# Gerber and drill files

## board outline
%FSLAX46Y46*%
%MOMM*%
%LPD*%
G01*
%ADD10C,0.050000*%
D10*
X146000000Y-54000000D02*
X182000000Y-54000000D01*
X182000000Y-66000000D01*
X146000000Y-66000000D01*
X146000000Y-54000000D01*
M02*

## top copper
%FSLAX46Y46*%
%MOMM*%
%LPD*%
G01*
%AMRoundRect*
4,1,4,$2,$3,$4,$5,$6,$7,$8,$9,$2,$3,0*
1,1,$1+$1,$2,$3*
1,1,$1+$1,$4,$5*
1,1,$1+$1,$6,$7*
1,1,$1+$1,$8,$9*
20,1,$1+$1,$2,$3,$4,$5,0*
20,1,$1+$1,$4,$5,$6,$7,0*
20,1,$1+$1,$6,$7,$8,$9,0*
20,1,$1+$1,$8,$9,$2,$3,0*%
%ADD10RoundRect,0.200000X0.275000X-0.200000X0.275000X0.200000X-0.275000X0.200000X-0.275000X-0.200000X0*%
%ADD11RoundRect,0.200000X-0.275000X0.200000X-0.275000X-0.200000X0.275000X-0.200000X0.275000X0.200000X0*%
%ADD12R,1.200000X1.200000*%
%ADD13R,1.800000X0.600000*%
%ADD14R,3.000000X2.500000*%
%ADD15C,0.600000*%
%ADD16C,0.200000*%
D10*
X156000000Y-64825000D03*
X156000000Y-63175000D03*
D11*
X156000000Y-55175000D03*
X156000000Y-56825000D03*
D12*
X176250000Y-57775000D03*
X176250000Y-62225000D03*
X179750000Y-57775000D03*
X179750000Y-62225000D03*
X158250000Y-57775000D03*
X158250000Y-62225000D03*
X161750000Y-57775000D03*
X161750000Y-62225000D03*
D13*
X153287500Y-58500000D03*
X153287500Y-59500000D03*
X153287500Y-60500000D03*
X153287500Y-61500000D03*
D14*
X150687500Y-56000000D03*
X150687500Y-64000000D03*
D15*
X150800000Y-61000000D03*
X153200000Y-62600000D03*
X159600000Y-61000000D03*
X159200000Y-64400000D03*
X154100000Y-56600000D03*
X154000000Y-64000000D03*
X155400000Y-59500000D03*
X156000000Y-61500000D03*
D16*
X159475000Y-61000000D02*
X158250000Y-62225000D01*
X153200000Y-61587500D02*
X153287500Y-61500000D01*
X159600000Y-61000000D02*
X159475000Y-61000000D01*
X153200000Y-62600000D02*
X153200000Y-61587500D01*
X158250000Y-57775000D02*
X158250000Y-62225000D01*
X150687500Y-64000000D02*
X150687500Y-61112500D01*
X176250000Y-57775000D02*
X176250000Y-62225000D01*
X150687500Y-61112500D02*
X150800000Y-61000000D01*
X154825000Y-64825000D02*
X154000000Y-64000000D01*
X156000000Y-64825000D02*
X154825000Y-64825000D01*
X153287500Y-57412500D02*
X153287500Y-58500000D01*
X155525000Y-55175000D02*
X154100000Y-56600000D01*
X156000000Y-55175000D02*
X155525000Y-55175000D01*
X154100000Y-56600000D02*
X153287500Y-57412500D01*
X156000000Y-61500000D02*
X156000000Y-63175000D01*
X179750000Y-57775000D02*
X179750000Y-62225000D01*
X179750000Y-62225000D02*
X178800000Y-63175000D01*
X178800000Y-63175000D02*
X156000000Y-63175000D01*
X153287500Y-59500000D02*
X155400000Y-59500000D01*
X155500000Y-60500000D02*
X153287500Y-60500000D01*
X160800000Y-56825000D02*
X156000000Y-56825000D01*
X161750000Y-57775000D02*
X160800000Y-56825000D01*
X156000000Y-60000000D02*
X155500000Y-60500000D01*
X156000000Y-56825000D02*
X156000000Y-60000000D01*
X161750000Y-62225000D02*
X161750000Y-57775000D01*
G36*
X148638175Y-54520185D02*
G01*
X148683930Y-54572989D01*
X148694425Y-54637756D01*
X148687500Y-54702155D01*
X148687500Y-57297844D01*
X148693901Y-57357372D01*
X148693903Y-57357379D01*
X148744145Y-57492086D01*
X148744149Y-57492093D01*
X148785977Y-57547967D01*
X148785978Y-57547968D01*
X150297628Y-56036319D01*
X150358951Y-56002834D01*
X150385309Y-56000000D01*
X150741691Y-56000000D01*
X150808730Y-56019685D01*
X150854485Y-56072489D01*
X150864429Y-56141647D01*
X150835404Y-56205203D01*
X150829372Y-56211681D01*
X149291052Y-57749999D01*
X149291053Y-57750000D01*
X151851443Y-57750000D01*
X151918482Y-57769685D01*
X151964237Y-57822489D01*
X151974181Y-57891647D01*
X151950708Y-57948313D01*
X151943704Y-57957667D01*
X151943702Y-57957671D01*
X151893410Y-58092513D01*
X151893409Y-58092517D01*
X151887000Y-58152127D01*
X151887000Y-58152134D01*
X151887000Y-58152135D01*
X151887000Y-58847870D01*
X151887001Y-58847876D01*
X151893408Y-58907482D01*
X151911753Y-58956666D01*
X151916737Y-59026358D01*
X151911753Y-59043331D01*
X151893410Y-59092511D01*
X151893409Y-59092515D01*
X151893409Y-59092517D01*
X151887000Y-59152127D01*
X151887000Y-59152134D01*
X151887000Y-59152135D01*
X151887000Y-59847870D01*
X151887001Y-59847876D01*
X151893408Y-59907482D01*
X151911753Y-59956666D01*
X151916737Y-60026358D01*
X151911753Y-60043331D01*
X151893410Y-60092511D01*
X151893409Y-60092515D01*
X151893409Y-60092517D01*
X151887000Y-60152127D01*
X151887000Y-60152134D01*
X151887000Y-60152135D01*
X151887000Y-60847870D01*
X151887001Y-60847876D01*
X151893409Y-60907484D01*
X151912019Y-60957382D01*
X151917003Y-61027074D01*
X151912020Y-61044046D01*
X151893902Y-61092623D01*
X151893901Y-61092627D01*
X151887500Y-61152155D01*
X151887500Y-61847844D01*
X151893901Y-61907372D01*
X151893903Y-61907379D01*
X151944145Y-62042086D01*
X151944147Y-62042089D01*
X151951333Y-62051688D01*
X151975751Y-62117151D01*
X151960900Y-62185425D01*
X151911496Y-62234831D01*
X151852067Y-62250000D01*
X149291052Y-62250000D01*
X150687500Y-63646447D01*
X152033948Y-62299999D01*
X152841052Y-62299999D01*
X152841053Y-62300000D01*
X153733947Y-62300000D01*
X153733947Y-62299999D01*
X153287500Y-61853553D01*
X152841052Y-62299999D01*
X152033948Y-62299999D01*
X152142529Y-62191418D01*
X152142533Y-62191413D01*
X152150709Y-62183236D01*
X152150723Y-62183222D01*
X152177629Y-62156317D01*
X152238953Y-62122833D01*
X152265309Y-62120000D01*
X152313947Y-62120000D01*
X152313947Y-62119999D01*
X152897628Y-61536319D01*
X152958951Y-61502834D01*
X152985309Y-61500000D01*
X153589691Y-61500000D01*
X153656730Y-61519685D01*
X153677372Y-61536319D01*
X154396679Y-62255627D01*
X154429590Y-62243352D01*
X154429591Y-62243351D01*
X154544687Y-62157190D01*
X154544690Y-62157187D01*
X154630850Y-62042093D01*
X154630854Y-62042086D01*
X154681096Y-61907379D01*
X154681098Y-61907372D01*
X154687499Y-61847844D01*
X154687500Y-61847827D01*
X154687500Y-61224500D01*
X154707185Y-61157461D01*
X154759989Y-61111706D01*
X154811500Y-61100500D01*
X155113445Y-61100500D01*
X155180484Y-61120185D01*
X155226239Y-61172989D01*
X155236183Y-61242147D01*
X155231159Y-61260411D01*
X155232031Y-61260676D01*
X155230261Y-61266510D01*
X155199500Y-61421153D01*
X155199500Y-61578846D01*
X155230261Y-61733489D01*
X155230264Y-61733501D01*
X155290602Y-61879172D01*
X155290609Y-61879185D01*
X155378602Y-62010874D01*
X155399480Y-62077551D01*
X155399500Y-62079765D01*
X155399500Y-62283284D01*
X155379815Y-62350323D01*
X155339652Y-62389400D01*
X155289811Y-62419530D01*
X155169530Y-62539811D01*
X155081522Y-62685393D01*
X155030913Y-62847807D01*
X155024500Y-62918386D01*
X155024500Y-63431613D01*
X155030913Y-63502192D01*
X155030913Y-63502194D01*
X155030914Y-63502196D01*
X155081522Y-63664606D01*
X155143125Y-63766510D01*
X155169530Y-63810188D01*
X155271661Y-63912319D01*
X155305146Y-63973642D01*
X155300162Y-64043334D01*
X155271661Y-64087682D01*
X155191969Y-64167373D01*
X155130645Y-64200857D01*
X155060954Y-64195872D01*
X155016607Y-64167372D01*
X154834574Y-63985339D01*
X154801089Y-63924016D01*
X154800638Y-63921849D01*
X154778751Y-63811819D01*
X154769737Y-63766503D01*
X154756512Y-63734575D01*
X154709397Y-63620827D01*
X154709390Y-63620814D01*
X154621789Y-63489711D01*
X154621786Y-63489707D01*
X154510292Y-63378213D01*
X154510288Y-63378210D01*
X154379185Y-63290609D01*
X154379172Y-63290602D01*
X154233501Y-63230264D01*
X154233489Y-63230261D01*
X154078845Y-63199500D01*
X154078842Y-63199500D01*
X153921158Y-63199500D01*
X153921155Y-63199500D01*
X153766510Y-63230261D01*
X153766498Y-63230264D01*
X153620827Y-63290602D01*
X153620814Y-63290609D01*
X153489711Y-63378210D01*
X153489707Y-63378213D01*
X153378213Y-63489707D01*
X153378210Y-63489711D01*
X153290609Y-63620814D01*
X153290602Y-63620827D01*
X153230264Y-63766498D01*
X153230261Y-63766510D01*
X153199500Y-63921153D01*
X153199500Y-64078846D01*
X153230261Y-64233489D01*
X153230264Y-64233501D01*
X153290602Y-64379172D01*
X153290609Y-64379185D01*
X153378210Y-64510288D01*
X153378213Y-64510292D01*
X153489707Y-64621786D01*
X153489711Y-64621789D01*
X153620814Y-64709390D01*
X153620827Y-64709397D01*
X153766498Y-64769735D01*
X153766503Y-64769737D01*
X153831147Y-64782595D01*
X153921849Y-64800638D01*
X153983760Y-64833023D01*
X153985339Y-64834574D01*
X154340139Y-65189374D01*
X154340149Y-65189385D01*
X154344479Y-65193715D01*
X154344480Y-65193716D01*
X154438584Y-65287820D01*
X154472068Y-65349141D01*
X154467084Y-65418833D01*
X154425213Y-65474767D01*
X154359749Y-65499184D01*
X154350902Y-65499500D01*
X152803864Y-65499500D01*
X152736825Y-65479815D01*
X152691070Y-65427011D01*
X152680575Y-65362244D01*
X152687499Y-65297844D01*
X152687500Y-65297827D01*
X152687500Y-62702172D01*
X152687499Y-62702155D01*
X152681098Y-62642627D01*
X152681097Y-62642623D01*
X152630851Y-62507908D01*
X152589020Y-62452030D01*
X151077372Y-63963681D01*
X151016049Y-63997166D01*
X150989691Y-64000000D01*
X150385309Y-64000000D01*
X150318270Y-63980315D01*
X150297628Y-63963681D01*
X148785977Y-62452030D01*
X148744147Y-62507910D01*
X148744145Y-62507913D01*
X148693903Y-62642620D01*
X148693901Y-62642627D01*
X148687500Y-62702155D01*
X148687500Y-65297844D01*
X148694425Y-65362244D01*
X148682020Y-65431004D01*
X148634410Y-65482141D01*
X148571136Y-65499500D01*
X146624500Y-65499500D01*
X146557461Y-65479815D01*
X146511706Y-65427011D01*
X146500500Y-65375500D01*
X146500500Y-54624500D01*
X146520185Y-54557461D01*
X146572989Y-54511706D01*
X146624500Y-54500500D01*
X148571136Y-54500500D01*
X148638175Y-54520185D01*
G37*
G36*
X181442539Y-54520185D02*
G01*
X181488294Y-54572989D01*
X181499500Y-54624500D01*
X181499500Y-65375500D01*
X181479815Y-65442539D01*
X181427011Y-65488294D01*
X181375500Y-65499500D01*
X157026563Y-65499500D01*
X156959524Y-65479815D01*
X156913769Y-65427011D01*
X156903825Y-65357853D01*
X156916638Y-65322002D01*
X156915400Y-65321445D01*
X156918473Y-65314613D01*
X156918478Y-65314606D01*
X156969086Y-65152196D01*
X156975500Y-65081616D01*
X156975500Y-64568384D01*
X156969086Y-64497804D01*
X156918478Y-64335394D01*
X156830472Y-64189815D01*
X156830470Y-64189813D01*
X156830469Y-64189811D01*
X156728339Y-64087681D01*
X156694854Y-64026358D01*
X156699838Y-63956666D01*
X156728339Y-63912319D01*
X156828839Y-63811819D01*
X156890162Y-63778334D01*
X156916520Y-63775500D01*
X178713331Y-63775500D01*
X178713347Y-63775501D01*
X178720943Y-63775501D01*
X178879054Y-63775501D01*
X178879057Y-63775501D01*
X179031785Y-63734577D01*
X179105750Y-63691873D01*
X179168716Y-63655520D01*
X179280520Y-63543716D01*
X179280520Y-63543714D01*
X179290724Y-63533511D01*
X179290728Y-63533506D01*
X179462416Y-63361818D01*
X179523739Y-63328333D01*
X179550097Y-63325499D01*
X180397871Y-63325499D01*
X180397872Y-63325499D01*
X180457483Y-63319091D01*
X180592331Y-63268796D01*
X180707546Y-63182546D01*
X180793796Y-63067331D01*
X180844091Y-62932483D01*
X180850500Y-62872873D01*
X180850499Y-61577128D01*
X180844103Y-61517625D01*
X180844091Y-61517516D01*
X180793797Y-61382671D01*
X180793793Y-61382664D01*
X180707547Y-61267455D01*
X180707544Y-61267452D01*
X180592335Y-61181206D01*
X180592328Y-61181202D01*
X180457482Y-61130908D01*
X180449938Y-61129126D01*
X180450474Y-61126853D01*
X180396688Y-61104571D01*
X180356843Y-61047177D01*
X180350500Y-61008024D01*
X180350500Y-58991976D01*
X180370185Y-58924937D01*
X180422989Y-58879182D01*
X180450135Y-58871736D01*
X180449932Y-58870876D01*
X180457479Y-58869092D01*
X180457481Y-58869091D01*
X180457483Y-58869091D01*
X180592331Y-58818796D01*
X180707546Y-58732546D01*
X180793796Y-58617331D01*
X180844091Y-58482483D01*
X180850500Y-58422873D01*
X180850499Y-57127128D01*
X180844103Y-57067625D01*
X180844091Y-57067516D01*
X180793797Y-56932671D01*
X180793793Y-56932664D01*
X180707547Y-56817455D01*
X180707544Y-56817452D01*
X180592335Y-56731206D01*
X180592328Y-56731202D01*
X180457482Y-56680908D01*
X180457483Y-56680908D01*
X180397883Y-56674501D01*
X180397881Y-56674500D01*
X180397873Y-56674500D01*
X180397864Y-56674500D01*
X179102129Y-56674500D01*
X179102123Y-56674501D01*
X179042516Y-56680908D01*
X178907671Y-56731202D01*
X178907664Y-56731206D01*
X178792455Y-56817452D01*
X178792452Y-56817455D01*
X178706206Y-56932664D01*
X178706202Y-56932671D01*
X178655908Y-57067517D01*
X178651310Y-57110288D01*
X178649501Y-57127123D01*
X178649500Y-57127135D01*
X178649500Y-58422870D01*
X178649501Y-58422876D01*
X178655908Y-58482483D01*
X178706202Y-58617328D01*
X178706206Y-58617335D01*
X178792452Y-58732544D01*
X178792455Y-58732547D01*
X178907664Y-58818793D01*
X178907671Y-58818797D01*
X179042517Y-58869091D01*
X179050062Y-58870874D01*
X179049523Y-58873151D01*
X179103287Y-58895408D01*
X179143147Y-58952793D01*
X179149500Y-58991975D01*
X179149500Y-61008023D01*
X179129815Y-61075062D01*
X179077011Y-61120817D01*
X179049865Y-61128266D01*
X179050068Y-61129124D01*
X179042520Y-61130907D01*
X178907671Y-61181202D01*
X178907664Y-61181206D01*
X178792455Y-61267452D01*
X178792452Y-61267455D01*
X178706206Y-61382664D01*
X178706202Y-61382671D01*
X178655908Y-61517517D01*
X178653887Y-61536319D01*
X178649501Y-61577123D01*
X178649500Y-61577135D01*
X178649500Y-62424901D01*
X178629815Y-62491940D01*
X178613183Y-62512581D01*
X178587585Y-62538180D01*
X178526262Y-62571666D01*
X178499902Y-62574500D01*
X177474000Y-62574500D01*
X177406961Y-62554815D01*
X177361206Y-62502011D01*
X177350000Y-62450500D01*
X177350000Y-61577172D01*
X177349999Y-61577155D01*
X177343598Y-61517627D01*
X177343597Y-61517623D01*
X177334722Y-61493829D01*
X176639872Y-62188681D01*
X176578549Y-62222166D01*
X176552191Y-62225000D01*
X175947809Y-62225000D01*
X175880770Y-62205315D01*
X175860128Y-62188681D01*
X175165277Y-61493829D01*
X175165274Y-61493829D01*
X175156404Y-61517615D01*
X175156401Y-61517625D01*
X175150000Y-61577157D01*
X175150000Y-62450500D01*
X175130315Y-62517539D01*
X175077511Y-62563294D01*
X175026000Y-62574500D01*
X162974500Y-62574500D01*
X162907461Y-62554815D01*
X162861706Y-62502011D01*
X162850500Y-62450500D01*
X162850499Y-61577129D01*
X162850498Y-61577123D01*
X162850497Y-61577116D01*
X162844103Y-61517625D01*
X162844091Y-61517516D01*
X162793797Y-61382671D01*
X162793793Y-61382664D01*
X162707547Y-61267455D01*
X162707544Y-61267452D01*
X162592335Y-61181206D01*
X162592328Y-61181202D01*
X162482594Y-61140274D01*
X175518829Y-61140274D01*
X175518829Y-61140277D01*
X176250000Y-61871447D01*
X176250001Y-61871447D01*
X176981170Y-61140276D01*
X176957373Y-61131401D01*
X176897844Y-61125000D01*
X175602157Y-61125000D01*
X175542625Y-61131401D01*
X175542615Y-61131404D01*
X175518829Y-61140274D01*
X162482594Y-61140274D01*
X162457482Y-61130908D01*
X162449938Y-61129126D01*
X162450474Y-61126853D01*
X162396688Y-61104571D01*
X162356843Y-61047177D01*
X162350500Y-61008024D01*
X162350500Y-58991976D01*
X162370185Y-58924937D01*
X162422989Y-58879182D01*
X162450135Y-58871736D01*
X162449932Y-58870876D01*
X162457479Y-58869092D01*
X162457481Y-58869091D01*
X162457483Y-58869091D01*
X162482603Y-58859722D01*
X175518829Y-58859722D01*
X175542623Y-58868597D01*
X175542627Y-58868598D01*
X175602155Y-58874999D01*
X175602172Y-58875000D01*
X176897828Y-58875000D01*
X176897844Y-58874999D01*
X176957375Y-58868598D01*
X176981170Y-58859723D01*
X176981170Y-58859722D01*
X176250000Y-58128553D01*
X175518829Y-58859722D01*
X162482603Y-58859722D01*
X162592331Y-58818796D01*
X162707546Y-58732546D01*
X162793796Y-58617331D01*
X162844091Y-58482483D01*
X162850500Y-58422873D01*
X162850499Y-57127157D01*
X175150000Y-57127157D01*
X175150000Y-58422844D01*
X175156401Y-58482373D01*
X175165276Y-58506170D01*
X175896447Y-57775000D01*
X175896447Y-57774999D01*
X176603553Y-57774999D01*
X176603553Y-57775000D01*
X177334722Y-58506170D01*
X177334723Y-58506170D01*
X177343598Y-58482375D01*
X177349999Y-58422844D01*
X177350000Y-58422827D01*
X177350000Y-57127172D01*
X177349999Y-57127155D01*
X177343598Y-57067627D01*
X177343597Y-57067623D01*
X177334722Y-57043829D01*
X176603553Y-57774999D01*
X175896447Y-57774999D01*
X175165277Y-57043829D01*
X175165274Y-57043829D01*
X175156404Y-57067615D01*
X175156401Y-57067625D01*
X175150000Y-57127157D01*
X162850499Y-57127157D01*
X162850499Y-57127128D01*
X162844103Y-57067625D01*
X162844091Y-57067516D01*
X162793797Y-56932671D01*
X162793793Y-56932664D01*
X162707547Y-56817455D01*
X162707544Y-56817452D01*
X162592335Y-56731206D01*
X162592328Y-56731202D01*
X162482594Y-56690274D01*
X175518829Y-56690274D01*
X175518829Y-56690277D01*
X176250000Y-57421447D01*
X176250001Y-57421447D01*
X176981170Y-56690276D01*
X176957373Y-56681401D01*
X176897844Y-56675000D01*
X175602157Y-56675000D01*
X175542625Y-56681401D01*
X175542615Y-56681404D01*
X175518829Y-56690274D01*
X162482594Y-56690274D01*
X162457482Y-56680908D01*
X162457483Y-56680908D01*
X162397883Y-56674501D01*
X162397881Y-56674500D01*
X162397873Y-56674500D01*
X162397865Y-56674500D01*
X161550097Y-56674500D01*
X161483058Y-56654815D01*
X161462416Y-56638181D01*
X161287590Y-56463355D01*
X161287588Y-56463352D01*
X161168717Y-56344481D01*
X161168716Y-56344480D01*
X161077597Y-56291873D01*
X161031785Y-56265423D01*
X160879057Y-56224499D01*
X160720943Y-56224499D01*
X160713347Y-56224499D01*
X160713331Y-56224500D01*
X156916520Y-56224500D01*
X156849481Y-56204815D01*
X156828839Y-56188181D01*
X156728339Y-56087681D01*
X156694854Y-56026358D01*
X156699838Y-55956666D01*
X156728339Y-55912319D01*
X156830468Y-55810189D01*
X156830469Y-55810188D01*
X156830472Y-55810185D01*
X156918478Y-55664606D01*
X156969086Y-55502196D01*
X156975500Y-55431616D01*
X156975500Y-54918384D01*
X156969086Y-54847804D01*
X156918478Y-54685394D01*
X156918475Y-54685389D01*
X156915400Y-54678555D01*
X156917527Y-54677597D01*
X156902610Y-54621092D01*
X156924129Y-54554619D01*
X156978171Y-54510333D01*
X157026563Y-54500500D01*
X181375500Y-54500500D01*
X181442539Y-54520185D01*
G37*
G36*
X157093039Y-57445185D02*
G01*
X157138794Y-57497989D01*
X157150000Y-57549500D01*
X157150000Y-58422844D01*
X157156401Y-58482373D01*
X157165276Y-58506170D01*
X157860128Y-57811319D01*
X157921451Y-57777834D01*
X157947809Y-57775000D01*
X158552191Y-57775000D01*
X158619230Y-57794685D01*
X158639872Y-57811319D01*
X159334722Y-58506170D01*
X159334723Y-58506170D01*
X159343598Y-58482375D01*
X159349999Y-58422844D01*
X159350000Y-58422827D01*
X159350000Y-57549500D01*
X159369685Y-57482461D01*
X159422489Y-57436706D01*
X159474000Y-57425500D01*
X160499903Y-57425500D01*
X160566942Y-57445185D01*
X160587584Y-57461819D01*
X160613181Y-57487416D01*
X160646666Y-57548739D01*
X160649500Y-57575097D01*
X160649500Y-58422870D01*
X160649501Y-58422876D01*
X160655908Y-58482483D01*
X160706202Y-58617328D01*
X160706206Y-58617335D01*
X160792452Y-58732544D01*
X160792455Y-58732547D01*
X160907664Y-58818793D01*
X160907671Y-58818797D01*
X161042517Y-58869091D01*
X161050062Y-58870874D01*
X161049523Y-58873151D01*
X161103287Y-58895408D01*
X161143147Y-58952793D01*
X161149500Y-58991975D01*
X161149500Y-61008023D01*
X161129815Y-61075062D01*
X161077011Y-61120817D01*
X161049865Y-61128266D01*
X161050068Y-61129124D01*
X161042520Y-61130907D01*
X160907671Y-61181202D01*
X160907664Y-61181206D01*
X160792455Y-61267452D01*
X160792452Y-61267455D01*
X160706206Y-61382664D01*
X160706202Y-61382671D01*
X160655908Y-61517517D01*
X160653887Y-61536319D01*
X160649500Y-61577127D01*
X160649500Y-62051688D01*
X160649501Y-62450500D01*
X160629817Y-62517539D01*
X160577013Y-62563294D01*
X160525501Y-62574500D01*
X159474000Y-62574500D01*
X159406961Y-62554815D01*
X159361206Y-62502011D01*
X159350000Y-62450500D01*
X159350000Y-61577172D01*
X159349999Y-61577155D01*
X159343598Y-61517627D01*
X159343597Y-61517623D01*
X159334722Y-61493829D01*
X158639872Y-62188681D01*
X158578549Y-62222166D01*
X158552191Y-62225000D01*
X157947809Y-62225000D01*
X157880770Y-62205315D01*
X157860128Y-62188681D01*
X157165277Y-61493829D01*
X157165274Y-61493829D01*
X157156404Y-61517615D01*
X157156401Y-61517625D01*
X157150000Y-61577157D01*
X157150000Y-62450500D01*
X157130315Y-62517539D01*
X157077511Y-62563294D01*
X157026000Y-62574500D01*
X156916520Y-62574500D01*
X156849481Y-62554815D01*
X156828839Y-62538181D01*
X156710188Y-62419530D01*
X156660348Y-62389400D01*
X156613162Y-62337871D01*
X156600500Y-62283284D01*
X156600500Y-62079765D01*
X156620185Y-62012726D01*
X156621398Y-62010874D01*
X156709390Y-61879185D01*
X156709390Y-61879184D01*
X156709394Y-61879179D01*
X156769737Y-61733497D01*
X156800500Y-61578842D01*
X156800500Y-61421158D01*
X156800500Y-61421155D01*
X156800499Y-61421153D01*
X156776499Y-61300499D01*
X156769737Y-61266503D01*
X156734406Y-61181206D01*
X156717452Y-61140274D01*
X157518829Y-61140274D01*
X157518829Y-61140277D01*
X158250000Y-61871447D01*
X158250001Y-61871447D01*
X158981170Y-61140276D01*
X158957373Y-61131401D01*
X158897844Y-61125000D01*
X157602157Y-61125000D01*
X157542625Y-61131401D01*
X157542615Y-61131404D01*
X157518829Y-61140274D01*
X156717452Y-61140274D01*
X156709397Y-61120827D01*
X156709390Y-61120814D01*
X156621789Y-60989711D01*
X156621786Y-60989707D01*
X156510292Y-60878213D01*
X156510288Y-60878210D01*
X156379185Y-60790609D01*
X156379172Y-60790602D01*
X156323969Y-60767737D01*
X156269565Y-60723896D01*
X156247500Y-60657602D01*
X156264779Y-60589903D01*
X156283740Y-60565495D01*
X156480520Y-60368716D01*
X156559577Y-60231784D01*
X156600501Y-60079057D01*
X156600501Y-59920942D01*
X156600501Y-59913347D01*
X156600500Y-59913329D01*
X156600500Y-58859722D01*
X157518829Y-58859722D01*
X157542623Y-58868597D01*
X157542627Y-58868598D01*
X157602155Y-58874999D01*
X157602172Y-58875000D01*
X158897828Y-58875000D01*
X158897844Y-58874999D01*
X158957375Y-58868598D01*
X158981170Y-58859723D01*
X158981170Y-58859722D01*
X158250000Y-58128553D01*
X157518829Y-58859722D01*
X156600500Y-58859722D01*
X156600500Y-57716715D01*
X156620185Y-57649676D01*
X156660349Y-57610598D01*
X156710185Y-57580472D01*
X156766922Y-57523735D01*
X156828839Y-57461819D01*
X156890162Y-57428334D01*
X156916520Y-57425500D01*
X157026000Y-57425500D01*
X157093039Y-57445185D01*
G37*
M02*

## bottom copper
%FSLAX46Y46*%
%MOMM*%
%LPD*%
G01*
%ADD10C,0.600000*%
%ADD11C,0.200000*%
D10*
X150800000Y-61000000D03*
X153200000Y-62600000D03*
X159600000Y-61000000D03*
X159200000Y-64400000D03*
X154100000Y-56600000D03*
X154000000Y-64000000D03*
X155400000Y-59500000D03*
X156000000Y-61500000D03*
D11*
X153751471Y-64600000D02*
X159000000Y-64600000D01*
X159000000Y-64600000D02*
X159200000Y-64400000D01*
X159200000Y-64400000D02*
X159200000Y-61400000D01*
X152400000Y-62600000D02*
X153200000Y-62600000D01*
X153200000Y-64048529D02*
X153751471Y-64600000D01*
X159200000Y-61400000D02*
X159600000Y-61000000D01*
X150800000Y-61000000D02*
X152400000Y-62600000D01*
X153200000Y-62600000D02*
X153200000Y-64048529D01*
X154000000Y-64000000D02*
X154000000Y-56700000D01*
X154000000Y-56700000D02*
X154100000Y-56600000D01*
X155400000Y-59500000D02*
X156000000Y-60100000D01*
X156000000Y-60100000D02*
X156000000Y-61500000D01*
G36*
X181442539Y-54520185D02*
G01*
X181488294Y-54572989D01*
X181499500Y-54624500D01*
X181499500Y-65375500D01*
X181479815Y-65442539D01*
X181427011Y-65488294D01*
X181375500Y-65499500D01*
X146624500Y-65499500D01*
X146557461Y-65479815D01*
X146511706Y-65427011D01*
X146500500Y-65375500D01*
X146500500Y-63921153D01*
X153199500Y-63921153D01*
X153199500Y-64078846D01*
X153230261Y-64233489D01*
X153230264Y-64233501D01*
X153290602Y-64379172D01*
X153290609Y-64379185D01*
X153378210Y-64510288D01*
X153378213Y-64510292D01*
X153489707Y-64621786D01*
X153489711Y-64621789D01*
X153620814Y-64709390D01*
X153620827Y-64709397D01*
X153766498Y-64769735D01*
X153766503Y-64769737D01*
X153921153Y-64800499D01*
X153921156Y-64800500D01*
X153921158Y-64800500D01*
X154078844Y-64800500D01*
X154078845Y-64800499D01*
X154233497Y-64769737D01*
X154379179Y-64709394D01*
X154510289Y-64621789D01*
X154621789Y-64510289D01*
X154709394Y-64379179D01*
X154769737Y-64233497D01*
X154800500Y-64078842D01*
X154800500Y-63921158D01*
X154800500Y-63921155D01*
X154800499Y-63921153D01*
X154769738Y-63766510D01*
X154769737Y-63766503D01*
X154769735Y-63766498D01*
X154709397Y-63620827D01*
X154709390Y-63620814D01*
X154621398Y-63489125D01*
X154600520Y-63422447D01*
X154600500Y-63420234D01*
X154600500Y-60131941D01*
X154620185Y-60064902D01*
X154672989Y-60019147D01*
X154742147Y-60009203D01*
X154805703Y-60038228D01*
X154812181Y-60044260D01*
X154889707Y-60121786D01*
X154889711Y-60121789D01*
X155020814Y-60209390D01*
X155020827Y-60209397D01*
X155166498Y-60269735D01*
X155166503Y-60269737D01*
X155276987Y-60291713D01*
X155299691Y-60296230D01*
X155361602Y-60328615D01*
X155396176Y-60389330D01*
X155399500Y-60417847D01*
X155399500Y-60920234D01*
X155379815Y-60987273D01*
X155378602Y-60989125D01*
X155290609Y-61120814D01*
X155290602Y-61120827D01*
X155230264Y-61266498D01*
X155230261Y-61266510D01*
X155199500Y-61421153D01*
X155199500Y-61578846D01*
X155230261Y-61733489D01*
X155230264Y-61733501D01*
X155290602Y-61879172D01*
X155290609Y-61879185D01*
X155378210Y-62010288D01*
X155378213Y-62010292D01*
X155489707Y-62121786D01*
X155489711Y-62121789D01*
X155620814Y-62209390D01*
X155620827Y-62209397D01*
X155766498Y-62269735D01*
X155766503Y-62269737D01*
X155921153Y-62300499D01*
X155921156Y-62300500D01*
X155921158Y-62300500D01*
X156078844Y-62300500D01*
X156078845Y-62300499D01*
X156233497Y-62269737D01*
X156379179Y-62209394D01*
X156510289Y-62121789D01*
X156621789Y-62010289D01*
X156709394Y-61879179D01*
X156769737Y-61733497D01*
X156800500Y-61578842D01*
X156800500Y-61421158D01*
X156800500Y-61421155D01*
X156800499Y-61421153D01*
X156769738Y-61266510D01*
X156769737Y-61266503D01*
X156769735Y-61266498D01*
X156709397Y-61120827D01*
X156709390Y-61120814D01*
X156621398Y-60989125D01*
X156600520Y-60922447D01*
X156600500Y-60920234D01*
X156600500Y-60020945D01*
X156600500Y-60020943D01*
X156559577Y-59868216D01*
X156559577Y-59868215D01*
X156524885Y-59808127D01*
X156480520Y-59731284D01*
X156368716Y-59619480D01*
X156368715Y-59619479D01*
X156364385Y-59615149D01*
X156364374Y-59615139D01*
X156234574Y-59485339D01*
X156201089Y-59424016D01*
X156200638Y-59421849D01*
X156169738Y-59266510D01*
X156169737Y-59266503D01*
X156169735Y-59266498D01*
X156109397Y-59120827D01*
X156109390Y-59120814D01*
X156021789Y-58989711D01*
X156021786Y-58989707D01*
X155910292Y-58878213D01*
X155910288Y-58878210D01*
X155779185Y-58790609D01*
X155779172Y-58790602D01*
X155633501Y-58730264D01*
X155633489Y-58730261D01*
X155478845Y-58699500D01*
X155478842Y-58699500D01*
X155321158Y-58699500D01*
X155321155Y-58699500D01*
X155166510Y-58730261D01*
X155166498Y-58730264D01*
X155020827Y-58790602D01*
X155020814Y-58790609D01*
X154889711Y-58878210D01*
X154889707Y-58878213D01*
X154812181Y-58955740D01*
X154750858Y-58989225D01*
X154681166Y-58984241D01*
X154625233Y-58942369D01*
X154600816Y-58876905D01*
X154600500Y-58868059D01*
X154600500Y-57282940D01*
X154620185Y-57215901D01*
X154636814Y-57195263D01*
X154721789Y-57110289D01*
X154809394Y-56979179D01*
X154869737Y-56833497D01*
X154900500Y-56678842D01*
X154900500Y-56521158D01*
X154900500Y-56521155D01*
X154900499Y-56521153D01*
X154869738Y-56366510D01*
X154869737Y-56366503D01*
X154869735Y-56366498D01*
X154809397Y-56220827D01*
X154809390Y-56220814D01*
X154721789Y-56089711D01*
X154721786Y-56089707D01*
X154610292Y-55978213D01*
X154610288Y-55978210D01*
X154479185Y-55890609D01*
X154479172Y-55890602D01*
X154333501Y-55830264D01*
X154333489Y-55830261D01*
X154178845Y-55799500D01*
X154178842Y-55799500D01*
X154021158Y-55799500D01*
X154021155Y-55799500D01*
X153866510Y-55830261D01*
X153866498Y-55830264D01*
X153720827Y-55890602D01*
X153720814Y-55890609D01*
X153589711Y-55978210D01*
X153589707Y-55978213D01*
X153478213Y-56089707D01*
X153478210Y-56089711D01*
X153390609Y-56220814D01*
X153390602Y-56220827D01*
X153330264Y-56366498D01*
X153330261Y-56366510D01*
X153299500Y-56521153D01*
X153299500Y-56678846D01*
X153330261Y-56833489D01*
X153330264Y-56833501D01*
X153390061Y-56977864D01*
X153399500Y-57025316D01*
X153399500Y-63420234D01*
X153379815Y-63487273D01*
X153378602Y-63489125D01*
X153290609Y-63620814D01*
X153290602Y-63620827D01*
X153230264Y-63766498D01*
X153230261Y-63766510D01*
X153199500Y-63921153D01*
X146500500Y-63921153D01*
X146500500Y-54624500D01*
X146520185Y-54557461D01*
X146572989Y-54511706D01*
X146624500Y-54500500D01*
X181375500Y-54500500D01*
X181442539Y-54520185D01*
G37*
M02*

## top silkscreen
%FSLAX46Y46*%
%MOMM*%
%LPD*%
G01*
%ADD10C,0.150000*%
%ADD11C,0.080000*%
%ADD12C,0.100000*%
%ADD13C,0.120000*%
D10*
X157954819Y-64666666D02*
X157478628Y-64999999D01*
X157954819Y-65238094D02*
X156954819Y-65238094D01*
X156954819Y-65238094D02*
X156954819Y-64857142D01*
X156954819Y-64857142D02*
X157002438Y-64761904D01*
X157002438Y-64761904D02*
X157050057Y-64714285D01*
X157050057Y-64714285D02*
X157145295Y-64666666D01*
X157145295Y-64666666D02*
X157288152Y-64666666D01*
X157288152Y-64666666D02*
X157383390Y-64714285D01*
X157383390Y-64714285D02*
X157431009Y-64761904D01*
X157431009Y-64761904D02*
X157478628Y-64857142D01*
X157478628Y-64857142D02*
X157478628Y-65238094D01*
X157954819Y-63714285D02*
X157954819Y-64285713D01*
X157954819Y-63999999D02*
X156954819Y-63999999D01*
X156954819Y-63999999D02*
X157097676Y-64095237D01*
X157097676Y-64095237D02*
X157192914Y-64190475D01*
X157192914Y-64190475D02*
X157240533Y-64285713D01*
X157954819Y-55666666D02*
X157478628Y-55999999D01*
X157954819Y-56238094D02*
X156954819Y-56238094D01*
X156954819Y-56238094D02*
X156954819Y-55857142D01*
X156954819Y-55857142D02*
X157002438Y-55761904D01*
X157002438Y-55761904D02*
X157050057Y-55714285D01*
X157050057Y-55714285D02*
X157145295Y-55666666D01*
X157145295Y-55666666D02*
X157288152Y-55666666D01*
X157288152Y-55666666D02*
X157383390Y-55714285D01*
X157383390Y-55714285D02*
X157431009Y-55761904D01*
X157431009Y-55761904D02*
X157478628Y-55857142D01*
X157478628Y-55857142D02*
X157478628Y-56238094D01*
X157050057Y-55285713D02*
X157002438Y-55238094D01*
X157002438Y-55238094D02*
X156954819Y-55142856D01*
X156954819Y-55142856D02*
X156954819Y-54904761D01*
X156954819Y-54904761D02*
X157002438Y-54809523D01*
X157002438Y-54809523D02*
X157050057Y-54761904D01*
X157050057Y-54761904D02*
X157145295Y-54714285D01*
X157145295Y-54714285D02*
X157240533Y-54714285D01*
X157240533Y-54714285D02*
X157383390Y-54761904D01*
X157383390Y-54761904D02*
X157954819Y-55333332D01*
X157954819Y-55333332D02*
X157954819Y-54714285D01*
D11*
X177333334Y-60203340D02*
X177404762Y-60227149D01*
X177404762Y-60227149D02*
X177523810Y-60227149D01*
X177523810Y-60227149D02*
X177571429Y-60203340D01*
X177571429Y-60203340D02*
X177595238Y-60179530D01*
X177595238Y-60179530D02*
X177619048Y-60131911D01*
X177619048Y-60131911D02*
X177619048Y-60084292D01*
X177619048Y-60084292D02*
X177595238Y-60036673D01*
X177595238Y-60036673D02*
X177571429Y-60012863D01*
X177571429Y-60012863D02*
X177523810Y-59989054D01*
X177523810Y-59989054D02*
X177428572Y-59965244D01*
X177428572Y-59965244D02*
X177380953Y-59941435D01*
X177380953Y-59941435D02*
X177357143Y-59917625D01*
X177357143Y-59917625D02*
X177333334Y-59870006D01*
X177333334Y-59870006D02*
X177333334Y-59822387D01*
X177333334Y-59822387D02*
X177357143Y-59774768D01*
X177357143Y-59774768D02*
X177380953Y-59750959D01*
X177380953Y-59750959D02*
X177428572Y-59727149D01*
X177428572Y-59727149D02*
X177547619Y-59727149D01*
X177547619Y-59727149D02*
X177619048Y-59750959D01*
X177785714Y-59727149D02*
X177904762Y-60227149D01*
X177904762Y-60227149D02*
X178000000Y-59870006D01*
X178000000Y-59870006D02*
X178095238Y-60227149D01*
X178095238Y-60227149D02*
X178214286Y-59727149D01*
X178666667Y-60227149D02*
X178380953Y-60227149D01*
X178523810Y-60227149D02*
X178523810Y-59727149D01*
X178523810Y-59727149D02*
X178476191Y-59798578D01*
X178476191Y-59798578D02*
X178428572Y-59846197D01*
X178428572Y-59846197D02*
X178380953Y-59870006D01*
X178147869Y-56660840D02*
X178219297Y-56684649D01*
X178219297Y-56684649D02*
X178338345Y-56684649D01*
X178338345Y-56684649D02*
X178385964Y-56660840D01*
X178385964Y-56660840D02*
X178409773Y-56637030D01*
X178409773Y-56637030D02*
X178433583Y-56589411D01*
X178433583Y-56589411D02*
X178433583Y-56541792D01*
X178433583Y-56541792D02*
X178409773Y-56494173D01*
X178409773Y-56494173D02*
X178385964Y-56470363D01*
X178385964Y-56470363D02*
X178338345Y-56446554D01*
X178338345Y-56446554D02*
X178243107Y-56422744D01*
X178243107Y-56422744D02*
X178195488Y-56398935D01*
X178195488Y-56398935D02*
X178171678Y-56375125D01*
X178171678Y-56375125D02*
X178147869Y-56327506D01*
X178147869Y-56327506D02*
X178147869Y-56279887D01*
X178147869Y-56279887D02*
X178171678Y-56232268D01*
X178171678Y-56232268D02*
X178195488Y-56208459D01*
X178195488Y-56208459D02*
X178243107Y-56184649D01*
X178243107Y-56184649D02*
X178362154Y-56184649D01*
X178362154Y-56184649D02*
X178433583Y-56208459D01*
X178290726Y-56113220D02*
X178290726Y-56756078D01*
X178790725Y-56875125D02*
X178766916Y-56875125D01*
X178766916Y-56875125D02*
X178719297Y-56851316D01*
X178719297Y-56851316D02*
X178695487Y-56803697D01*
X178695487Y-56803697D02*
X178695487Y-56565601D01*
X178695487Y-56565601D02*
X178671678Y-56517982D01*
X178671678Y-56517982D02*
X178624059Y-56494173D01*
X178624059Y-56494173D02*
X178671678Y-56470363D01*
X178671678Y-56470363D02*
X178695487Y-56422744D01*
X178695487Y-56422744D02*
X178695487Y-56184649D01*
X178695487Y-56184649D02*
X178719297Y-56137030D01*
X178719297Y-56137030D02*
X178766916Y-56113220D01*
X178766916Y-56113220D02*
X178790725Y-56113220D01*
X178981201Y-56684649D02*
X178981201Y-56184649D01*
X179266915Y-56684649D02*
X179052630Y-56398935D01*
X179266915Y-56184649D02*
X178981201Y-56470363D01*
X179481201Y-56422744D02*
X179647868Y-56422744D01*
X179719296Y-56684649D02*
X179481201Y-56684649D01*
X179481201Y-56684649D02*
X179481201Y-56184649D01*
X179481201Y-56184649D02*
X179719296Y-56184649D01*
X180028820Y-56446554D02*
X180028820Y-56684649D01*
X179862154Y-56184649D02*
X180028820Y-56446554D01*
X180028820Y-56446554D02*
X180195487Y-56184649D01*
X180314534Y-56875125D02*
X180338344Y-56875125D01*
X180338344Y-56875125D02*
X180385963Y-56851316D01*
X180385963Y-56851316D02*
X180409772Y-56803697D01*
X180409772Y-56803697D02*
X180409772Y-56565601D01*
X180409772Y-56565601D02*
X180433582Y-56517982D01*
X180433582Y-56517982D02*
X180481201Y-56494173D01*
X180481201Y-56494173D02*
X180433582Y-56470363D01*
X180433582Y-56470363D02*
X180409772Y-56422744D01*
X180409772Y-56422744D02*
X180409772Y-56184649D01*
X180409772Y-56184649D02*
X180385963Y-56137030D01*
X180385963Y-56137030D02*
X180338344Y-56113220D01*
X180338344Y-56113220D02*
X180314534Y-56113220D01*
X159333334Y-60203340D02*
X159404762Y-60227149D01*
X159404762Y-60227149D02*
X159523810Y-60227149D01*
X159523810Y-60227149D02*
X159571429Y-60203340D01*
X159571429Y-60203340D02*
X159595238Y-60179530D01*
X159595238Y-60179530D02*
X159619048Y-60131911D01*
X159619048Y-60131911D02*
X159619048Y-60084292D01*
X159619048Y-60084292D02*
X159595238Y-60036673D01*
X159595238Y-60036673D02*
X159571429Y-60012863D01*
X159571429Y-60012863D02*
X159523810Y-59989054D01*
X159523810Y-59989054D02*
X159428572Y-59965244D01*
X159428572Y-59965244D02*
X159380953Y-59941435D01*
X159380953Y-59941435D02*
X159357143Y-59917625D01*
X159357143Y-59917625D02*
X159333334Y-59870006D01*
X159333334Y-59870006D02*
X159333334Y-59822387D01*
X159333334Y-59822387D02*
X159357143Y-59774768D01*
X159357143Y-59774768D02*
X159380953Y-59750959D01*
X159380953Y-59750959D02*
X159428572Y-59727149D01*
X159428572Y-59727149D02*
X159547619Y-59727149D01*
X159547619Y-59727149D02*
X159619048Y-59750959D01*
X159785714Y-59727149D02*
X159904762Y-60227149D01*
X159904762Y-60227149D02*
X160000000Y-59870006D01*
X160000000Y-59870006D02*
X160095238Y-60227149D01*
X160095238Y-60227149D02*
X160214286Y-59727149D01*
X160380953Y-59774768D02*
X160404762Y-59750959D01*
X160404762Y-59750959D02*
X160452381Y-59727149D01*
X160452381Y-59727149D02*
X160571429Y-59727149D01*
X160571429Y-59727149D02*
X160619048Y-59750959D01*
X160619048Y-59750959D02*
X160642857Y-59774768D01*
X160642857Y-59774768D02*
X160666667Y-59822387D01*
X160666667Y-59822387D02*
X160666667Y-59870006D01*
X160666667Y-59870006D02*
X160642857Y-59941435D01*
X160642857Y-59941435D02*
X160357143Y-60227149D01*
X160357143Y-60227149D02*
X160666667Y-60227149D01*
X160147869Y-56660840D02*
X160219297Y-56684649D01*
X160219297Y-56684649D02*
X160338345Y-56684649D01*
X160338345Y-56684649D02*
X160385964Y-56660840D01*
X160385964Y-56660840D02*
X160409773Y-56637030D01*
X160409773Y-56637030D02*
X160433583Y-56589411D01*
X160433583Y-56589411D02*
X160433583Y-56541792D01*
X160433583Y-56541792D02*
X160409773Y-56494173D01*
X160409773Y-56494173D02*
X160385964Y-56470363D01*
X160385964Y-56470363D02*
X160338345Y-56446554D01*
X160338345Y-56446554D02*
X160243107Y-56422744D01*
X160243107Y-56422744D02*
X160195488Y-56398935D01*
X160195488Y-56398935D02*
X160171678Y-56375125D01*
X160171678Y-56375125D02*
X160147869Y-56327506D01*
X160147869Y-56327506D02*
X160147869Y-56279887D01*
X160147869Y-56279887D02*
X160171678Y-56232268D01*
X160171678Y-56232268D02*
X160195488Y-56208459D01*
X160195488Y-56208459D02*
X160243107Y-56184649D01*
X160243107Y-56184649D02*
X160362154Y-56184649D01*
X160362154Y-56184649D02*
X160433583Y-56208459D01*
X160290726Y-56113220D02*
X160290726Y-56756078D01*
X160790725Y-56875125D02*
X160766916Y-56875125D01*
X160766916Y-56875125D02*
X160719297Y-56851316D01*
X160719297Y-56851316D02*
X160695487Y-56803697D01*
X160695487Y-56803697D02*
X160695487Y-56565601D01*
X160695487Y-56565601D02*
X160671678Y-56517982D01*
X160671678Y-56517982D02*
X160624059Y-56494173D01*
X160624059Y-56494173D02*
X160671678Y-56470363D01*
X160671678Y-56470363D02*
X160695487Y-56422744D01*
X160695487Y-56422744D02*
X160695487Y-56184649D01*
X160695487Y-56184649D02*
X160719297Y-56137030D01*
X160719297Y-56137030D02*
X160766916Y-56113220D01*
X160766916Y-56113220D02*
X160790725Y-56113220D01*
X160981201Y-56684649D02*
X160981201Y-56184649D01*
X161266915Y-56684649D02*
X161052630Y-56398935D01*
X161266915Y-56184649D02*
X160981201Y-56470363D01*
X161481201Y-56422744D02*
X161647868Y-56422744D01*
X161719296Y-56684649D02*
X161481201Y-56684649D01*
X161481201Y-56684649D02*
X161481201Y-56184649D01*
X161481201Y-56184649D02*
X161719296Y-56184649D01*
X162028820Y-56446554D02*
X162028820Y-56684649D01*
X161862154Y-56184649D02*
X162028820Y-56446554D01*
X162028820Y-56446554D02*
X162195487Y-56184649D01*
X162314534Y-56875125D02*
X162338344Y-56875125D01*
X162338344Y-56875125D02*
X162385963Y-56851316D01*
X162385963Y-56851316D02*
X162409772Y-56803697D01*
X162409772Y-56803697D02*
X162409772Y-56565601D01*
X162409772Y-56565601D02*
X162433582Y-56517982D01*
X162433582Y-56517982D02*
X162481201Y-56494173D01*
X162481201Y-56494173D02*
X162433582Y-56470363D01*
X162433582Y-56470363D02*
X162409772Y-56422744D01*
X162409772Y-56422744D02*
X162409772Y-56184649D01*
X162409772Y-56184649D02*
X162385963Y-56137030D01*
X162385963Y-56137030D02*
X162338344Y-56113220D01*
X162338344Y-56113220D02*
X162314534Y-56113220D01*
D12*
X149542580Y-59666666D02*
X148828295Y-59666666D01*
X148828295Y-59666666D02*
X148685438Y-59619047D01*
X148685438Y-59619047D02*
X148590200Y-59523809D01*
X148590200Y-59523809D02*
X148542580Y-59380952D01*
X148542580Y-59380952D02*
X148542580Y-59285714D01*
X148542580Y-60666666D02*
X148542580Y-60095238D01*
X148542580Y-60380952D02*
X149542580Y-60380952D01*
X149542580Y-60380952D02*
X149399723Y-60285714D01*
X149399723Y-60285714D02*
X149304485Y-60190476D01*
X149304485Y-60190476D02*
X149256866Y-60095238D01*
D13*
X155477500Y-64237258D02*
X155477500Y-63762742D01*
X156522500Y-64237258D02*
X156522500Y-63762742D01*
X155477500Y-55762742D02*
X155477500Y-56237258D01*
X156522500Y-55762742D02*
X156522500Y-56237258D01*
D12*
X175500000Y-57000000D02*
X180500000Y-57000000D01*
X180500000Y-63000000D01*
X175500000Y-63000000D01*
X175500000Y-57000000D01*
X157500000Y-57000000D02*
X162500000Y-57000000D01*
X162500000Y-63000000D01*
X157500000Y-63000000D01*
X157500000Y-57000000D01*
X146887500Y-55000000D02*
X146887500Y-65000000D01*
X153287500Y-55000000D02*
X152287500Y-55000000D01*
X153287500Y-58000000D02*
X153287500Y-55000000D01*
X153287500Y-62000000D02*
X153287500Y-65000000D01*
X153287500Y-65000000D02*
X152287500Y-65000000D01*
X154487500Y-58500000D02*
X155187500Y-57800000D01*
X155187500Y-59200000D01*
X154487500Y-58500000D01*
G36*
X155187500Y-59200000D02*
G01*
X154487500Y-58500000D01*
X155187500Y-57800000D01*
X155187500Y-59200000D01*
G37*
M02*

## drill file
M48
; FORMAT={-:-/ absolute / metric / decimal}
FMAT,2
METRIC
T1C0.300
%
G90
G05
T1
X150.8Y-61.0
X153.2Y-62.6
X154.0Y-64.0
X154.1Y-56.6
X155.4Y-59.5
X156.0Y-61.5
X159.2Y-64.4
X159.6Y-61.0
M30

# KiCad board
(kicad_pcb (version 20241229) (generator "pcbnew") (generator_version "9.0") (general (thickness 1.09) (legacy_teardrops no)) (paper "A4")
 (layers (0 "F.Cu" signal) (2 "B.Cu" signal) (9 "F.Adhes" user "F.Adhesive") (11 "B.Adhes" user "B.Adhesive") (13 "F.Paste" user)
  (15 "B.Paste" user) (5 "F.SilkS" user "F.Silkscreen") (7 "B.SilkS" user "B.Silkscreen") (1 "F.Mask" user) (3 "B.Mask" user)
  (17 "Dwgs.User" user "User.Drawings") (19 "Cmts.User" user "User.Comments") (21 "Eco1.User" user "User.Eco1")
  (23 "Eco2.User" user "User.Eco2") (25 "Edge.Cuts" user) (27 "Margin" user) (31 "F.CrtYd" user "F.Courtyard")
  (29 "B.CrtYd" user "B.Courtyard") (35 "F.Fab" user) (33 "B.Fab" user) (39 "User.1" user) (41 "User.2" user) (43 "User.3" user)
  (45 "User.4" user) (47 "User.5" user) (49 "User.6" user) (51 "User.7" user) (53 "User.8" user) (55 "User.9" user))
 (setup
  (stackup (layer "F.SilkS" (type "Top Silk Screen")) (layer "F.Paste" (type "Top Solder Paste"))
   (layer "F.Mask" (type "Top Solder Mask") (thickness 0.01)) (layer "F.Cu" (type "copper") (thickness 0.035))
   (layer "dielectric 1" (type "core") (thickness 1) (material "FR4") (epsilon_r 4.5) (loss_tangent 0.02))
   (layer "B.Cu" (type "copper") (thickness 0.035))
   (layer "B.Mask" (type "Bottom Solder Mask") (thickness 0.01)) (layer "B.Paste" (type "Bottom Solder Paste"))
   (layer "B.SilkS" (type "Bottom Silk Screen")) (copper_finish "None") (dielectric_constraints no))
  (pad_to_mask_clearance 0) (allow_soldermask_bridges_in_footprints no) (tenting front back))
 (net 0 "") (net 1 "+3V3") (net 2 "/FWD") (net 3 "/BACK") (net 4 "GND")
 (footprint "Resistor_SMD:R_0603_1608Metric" (layer "F.Cu") (at 156 64 90)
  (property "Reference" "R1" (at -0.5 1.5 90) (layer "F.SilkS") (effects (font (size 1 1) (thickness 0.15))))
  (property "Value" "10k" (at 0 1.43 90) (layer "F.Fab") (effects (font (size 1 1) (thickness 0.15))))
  (fp_line (start -0.237258 -0.5225) (end 0.237258 -0.5225) (stroke (width 0.12) (type solid)) (layer "F.SilkS"))
  (fp_line (start -0.237258 0.5225) (end 0.237258 0.5225) (stroke (width 0.12) (type solid)) (layer "F.SilkS"))
  (pad "1" smd roundrect (at -0.825 0 90) (size 0.8 0.95) (layers "F.Cu" "F.Mask" "F.Paste") (roundrect_rratio 0.25) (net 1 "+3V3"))
  (pad "2" smd roundrect (at 0.825 0 90) (size 0.8 0.95) (layers "F.Cu" "F.Mask" "F.Paste") (roundrect_rratio 0.25) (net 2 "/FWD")))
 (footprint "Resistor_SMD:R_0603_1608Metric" (layer "F.Cu") (at 156 56 -90)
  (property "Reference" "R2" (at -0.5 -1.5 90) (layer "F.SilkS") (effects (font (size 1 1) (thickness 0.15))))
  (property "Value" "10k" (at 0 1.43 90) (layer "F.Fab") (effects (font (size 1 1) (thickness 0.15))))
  (fp_line (start -0.237258 0.5225) (end 0.237258 0.5225) (stroke (width 0.12) (type solid)) (layer "F.SilkS"))
  (fp_line (start -0.237258 -0.5225) (end 0.237258 -0.5225) (stroke (width 0.12) (type solid)) (layer "F.SilkS"))
  (pad "1" smd roundrect (at -0.825 0 270) (size 0.8 0.95) (layers "F.Cu" "F.Mask" "F.Paste") (roundrect_rratio 0.25) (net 1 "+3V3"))
  (pad "2" smd roundrect (at 0.825 0 270) (size 0.8 0.95) (layers "F.Cu" "F.Mask" "F.Paste") (roundrect_rratio 0.25) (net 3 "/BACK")))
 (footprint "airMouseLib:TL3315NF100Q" (layer "F.Cu") (at 178 60)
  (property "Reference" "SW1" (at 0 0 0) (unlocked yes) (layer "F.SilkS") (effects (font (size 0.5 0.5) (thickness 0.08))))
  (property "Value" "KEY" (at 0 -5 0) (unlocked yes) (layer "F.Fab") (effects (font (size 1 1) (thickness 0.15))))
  (fp_rect (start -2.5 -3) (end 2.5 3) (stroke (width 0.1) (type default)) (fill no) (layer "F.SilkS"))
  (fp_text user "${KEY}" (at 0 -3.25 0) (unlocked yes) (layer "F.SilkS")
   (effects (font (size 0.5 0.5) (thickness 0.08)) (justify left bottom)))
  (pad "1" smd rect (at -1.75 -2.225) (size 1.2 1.2) (layers "F.Cu" "F.Mask" "F.Paste") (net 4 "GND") (thermal_bridge_angle 45))
  (pad "1" smd rect (at -1.75 2.225 180) (size 1.2 1.2) (layers "F.Cu" "F.Mask" "F.Paste") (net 4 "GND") (thermal_bridge_angle 45))
  (pad "2" smd rect (at 1.75 -2.225) (size 1.2 1.2) (layers "F.Cu" "F.Mask" "F.Paste") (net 2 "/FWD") (thermal_bridge_angle 45))
  (pad "2" smd rect (at 1.75 2.225 180) (size 1.2 1.2) (layers "F.Cu" "F.Mask" "F.Paste") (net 2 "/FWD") (thermal_bridge_angle 45)))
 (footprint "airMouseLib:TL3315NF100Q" (layer "F.Cu") (at 160 60)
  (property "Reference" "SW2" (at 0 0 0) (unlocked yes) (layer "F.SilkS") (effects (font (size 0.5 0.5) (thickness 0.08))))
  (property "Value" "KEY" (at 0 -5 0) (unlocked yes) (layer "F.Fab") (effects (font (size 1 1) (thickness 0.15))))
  (fp_rect (start -2.5 -3) (end 2.5 3) (stroke (width 0.1) (type default)) (fill no) (layer "F.SilkS"))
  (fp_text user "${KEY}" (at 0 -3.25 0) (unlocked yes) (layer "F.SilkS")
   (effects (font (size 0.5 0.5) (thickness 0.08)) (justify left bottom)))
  (pad "1" smd rect (at -1.75 -2.225) (size 1.2 1.2) (layers "F.Cu" "F.Mask" "F.Paste") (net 4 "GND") (thermal_bridge_angle 45))
  (pad "1" smd rect (at -1.75 2.225 180) (size 1.2 1.2) (layers "F.Cu" "F.Mask" "F.Paste") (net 4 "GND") (thermal_bridge_angle 45))
  (pad "2" smd rect (at 1.75 -2.225) (size 1.2 1.2) (layers "F.Cu" "F.Mask" "F.Paste") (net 3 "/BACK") (thermal_bridge_angle 45))
  (pad "2" smd rect (at 1.75 2.225 180) (size 1.2 1.2) (layers "F.Cu" "F.Mask" "F.Paste") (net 3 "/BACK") (thermal_bridge_angle 45)))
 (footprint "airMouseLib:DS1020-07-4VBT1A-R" (layer "F.Cu") (at 153.2875 60 -90)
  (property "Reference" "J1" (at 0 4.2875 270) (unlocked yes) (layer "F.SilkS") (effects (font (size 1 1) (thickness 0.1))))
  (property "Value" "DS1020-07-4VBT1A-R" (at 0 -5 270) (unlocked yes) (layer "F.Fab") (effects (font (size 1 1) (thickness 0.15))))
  (fp_line (start -5 6.4) (end 5 6.4) (stroke (width 0.1) (type default)) (layer "F.SilkS"))
  (fp_line (start -5 0) (end -5 1) (stroke (width 0.1) (type default)) (layer "F.SilkS"))
  (fp_line (start -2 0) (end -5 0) (stroke (width 0.1) (type default)) (layer "F.SilkS"))
  (fp_line (start 2 0) (end 5 0) (stroke (width 0.1) (type default)) (layer "F.SilkS"))
  (fp_line (start 5 0) (end 5 1) (stroke (width 0.1) (type default)) (layer "F.SilkS"))
  (fp_poly (pts (xy -1.5 -1.2) (xy -2.2 -1.9) (xy -0.8 -1.9)) (stroke (width 0.1) (type solid)) (fill yes) (layer "F.SilkS"))
  (pad "1" smd rect (at -1.5 0 270) (size 0.6 1.8) (layers "F.Cu" "F.Mask" "F.Paste") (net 1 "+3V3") (thermal_bridge_angle 45))
  (pad "2" smd rect (at -0.5 0 270) (size 0.6 1.8) (layers "F.Cu" "F.Mask" "F.Paste") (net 2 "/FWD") (thermal_bridge_angle 45))
  (pad "3" smd rect (at 0.5 0 270) (size 0.6 1.8) (layers "F.Cu" "F.Mask" "F.Paste") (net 3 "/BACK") (thermal_bridge_angle 45))
  (pad "4" smd rect (at 1.5 0 270) (size 0.6 1.8) (layers "F.Cu" "F.Mask" "F.Paste") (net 4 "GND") (thermal_bridge_angle 45))
  (pad "MP" smd rect (at -4 2.6 270) (size 2.5 3) (layers "F.Cu" "F.Mask" "F.Paste") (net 4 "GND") (thermal_bridge_angle 45))
  (pad "MP" smd rect (at 4 2.6 270) (size 2.5 3) (layers "F.Cu" "F.Mask" "F.Paste") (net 4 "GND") (thermal_bridge_angle 45)))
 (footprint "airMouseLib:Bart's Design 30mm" (layer "B.Cu") (at 163.8 60.4 180)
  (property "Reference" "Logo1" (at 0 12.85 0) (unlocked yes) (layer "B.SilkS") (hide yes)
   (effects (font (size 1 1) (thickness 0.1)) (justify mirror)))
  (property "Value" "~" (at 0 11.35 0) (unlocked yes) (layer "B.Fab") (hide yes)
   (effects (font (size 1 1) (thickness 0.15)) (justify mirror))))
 (gr_rect (start 146 54) (end 182 66) (stroke (width 0.05) (type default)) (fill no) (layer "Edge.Cuts"))
 (segment (start 159.475 61) (end 158.25 62.225) (width 0.2) (layer "F.Cu") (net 4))
 (segment (start 153.2 61.5875) (end 153.2875 61.5) (width 0.2) (layer "F.Cu") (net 4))
 (segment (start 159.6 61) (end 159.475 61) (width 0.2) (layer "F.Cu") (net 4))
 (segment (start 153.2 62.6) (end 153.2 61.5875) (width 0.2) (layer "F.Cu") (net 4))
 (segment (start 158.25 57.775) (end 158.25 62.225) (width 0.2) (layer "F.Cu") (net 4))
 (segment (start 150.6875 64) (end 150.6875 61.1125) (width 0.2) (layer "F.Cu") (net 4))
 (segment (start 176.25 57.775) (end 176.25 62.225) (width 0.2) (layer "F.Cu") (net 4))
 (segment (start 150.6875 61.1125) (end 150.8 61) (width 0.2) (layer "F.Cu") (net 4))
 (via (at 150.8 61) (size 0.6) (drill 0.3) (layers "F.Cu" "B.Cu") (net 4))
 (via (at 153.2 62.6) (size 0.6) (drill 0.3) (layers "F.Cu" "B.Cu") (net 4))
 (via (at 159.6 61) (size 0.6) (drill 0.3) (layers "F.Cu" "B.Cu") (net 4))
 (via (at 159.2 64.4) (size 0.6) (drill 0.3) (layers "F.Cu" "B.Cu") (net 4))
 (segment (start 153.751471 64.6) (end 159 64.6) (width 0.2) (layer "B.Cu") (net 4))
 (segment (start 159 64.6) (end 159.2 64.4) (width 0.2) (layer "B.Cu") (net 4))
 (segment (start 159.2 64.4) (end 159.2 61.4) (width 0.2) (layer "B.Cu") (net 4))
 (segment (start 152.4 62.6) (end 153.2 62.6) (width 0.2) (layer "B.Cu") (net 4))
 (segment (start 153.2 64.048529) (end 153.751471 64.6) (width 0.2) (layer "B.Cu") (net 4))
 (segment (start 159.2 61.4) (end 159.6 61) (width 0.2) (layer "B.Cu") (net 4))
 (segment (start 150.8 61) (end 152.4 62.6) (width 0.2) (layer "B.Cu") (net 4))
 (segment (start 153.2 62.6) (end 153.2 64.048529) (width 0.2) (layer "B.Cu") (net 4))
 (segment (start 154.825 64.825) (end 154 64) (width 0.2) (layer "F.Cu") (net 1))
 (segment (start 156 64.825) (end 154.825 64.825) (width 0.2) (layer "F.Cu") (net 1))
 (segment (start 153.2875 57.4125) (end 153.2875 58.5) (width 0.2) (layer "F.Cu") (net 1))
 (segment (start 155.525 55.175) (end 154.1 56.6) (width 0.2) (layer "F.Cu") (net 1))
 (segment (start 156 55.175) (end 155.525 55.175) (width 0.2) (layer "F.Cu") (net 1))
 (segment (start 154.1 56.6) (end 153.2875 57.4125) (width 0.2) (layer "F.Cu") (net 1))
 (via (at 154.1 56.6) (size 0.6) (drill 0.3) (layers "F.Cu" "B.Cu") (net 1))
 (via (at 154 64) (size 0.6) (drill 0.3) (layers "F.Cu" "B.Cu") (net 1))
 (segment (start 154 64) (end 154 56.7) (width 0.2) (layer "B.Cu") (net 1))
 (segment (start 154 56.7) (end 154.1 56.6) (width 0.2) (layer "B.Cu") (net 1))
 (segment (start 156 61.5) (end 156 63.175) (width 0.2) (layer "F.Cu") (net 2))
 (segment (start 179.75 57.775) (end 179.75 62.225) (width 0.2) (layer "F.Cu") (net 2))
 (segment (start 179.75 62.225) (end 178.8 63.175) (width 0.2) (layer "F.Cu") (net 2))
 (segment (start 178.8 63.175) (end 156 63.175) (width 0.2) (layer "F.Cu") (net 2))
 (segment (start 153.2875 59.5) (end 155.4 59.5) (width 0.2) (layer "F.Cu") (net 2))
 (via (at 155.4 59.5) (size 0.6) (drill 0.3) (layers "F.Cu" "B.Cu") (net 2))
 (via (at 156 61.5) (size 0.6) (drill 0.3) (layers "F.Cu" "B.Cu") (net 2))
 (segment (start 155.4 59.5) (end 156 60.1) (width 0.2) (layer "B.Cu") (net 2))
 (segment (start 156 60.1) (end 156 61.5) (width 0.2) (layer "B.Cu") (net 2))
 (segment (start 155.5 60.5) (end 153.2875 60.5) (width 0.2) (layer "F.Cu") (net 3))
 (segment (start 160.8 56.825) (end 156 56.825) (width 0.2) (layer "F.Cu") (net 3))
 (segment (start 161.75 57.775) (end 160.8 56.825) (width 0.2) (layer "F.Cu") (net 3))
 (segment (start 156 60) (end 155.5 60.5) (width 0.2) (layer "F.Cu") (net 3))
 (segment (start 156 56.825) (end 156 60) (width 0.2) (layer "F.Cu") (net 3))
 (segment (start 161.75 62.225) (end 161.75 57.775) (width 0.2) (layer "F.Cu") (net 3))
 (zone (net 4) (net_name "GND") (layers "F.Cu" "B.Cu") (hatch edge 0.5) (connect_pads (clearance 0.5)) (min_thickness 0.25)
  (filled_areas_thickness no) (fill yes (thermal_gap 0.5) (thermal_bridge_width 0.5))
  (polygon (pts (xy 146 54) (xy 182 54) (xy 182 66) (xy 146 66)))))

